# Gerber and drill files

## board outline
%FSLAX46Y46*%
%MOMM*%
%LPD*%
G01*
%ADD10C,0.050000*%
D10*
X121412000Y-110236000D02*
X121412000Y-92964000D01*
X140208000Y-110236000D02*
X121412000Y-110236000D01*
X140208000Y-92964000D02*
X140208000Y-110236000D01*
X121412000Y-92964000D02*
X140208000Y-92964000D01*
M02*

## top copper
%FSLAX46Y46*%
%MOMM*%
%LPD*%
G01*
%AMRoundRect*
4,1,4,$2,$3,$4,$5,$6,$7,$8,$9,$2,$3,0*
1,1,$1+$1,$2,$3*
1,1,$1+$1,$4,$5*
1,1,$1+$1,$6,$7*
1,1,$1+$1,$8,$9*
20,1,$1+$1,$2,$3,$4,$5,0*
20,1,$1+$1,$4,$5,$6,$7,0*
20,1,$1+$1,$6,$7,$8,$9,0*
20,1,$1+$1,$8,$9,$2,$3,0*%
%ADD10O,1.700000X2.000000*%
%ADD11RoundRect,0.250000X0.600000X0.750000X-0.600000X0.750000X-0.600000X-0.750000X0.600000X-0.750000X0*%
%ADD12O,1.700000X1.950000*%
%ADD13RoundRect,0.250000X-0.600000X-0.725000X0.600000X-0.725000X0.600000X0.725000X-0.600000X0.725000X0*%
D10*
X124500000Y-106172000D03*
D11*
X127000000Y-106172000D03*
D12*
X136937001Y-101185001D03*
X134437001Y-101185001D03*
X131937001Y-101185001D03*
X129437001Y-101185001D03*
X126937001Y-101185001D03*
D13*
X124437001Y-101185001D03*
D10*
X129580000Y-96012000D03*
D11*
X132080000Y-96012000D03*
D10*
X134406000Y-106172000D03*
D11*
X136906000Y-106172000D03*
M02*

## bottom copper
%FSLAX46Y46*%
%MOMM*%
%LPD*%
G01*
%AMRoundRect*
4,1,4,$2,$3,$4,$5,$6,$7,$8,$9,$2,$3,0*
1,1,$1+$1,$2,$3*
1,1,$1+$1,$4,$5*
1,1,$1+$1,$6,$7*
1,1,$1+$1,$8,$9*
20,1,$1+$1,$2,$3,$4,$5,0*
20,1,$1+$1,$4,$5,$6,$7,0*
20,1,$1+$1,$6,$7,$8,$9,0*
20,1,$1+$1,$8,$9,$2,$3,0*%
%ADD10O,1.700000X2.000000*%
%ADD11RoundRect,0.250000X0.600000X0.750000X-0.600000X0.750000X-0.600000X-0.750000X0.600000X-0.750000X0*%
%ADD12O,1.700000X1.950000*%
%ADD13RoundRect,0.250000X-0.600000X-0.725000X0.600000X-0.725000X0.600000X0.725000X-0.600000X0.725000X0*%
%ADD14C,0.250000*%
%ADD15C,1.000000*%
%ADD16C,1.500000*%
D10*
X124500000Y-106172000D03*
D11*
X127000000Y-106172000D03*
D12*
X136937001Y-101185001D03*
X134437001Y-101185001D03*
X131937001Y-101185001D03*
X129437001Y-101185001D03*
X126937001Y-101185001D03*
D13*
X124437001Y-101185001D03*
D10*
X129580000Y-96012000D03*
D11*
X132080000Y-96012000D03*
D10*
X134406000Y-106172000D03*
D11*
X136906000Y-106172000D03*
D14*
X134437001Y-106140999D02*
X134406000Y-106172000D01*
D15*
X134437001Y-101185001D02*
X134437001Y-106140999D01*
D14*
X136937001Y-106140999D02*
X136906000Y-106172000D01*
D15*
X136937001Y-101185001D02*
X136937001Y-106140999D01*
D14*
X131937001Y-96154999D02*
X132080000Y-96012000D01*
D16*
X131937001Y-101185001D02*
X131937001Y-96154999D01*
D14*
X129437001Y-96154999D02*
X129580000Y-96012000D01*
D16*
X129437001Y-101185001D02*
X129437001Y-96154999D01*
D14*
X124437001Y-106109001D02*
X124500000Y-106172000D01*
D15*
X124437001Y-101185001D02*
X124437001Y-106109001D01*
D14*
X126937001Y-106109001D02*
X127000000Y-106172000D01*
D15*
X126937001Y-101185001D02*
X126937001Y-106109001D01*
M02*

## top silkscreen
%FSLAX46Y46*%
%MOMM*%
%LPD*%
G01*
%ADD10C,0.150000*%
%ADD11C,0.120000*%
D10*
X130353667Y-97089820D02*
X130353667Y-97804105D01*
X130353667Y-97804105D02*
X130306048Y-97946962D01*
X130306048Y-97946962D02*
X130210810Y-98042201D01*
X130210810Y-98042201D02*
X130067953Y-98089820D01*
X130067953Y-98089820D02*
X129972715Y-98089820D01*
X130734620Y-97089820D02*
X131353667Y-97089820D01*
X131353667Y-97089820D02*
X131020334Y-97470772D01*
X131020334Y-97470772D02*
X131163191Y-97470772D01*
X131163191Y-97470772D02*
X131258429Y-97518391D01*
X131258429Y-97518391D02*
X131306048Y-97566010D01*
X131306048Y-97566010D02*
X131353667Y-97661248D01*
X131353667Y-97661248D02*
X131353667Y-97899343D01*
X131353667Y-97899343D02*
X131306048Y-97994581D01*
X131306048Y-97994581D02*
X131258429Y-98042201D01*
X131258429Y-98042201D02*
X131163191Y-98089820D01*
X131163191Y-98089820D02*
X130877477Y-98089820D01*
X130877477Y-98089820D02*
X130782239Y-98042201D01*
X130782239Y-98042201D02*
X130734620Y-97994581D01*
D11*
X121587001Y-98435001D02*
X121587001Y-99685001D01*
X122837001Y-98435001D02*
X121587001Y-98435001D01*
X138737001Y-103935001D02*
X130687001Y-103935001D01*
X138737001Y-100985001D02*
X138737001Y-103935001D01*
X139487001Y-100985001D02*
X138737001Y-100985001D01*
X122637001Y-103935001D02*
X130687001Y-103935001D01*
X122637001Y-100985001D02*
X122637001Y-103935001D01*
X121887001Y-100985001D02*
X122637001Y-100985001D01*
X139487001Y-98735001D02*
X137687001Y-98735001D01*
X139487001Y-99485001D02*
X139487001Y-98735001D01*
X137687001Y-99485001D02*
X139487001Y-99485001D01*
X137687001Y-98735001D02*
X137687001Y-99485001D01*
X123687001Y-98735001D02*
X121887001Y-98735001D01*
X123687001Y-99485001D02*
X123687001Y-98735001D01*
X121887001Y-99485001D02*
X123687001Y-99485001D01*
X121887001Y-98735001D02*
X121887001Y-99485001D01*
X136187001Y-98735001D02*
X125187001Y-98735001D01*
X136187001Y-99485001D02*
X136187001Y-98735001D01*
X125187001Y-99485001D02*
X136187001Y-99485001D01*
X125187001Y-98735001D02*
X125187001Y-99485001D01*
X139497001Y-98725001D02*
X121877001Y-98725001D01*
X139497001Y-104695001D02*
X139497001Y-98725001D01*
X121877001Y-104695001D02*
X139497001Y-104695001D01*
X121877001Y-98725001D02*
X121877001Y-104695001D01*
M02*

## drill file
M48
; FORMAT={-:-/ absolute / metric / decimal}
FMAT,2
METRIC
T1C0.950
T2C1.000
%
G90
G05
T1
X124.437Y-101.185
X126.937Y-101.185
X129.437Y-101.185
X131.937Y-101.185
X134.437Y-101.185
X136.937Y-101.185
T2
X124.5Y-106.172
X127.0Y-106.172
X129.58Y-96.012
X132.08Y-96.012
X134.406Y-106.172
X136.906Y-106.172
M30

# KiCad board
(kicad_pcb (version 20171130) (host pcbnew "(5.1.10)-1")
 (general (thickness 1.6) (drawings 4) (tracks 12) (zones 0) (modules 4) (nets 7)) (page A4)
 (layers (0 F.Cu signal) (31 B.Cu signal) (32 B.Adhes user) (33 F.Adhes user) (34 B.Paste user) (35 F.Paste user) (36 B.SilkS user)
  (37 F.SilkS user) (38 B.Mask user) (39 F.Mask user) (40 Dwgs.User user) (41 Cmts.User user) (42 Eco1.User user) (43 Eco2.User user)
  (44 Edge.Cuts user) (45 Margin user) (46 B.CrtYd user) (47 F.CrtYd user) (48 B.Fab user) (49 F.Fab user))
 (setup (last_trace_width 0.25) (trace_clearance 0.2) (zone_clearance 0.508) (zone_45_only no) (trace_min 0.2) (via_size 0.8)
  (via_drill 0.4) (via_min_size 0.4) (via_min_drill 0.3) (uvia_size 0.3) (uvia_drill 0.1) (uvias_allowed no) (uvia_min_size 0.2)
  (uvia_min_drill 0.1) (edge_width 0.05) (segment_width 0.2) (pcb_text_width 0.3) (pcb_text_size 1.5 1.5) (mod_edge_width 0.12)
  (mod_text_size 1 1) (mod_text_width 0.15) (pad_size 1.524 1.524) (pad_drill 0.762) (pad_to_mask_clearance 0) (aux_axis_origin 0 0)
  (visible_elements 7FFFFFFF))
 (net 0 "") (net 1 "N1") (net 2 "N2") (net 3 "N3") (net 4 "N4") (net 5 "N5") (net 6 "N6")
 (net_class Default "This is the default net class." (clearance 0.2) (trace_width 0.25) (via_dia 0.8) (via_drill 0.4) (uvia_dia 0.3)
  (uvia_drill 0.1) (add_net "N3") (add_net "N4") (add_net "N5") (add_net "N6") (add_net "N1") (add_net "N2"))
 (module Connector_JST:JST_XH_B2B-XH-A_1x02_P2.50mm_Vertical (layer B.Cu) (at 127 106.172 180)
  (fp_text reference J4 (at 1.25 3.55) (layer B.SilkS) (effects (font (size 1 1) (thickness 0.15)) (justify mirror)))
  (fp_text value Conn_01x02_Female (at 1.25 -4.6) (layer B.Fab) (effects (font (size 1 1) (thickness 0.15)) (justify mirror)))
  (pad 2 thru_hole oval (at 2.5 0 180) (size 1.7 2) (drill 1) (layers *.Cu *.Mask) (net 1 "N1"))
  (pad 1 thru_hole roundrect (at 0 0 180) (size 1.7 2) (drill 1) (layers *.Cu *.Mask) (roundrect_rratio 0.1470588235294118) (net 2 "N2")))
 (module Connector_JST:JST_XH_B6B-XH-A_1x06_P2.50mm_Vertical (layer F.Cu) (at 124.437001 101.185001)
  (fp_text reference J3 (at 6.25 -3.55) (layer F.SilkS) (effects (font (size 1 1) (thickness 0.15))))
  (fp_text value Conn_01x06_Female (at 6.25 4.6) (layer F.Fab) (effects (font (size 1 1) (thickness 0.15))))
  (fp_line (start -2.85 -2.75) (end -2.85 -1.5) (layer F.SilkS) (width 0.12))
  (fp_line (start -1.6 -2.75) (end -2.85 -2.75) (layer F.SilkS) (width 0.12))
  (fp_line (start 14.3 2.75) (end 6.25 2.75) (layer F.SilkS) (width 0.12))
  (fp_line (start 14.3 -0.2) (end 14.3 2.75) (layer F.SilkS) (width 0.12))
  (fp_line (start 15.05 -0.2) (end 14.3 -0.2) (layer F.SilkS) (width 0.12))
  (fp_line (start -1.8 2.75) (end 6.25 2.75) (layer F.SilkS) (width 0.12))
  (fp_line (start -1.8 -0.2) (end -1.8 2.75) (layer F.SilkS) (width 0.12))
  (fp_line (start -2.55 -0.2) (end -1.8 -0.2) (layer F.SilkS) (width 0.12))
  (fp_line (start 15.05 -2.45) (end 13.25 -2.45) (layer F.SilkS) (width 0.12))
  (fp_line (start 15.05 -1.7) (end 15.05 -2.45) (layer F.SilkS) (width 0.12))
  (fp_line (start 13.25 -1.7) (end 15.05 -1.7) (layer F.SilkS) (width 0.12))
  (fp_line (start 13.25 -2.45) (end 13.25 -1.7) (layer F.SilkS) (width 0.12))
  (fp_line (start -0.75 -2.45) (end -2.55 -2.45) (layer F.SilkS) (width 0.12))
  (fp_line (start -0.75 -1.7) (end -0.75 -2.45) (layer F.SilkS) (width 0.12))
  (fp_line (start -2.55 -1.7) (end -0.75 -1.7) (layer F.SilkS) (width 0.12))
  (fp_line (start -2.55 -2.45) (end -2.55 -1.7) (layer F.SilkS) (width 0.12))
  (fp_line (start 11.75 -2.45) (end 0.75 -2.45) (layer F.SilkS) (width 0.12))
  (fp_line (start 11.75 -1.7) (end 11.75 -2.45) (layer F.SilkS) (width 0.12))
  (fp_line (start 0.75 -1.7) (end 11.75 -1.7) (layer F.SilkS) (width 0.12))
  (fp_line (start 0.75 -2.45) (end 0.75 -1.7) (layer F.SilkS) (width 0.12))
  (fp_line (start 15.06 -2.46) (end -2.56 -2.46) (layer F.SilkS) (width 0.12))
  (fp_line (start 15.06 3.51) (end 15.06 -2.46) (layer F.SilkS) (width 0.12))
  (fp_line (start -2.56 3.51) (end 15.06 3.51) (layer F.SilkS) (width 0.12))
  (fp_line (start -2.56 -2.46) (end -2.56 3.51) (layer F.SilkS) (width 0.12))
  (pad 6 thru_hole oval (at 12.5 0) (size 1.7 1.95) (drill 0.95) (layers *.Cu *.Mask) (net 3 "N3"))
  (pad 5 thru_hole oval (at 10 0) (size 1.7 1.95) (drill 0.95) (layers *.Cu *.Mask) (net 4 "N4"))
  (pad 4 thru_hole oval (at 7.5 0) (size 1.7 1.95) (drill 0.95) (layers *.Cu *.Mask) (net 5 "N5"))
  (pad 3 thru_hole oval (at 5 0) (size 1.7 1.95) (drill 0.95) (layers *.Cu *.Mask) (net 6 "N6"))
  (pad 2 thru_hole oval (at 2.5 0) (size 1.7 1.95) (drill 0.95) (layers *.Cu *.Mask) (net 2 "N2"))
  (pad 1 thru_hole roundrect (at 0 0) (size 1.7 1.95) (drill 0.95) (layers *.Cu *.Mask) (roundrect_rratio 0.1470588235294118) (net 1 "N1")))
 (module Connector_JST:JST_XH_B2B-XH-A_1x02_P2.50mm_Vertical (layer B.Cu) (at 132.08 96.012 180)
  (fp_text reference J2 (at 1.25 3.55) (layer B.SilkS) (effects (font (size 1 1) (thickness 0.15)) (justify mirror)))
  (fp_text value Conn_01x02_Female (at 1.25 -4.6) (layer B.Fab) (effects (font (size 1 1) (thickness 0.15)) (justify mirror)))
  (pad 2 thru_hole oval (at 2.5 0 180) (size 1.7 2) (drill 1) (layers *.Cu *.Mask) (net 6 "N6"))
  (pad 1 thru_hole roundrect (at 0 0 180) (size 1.7 2) (drill 1) (layers *.Cu *.Mask) (roundrect_rratio 0.1470588235294118) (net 5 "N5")))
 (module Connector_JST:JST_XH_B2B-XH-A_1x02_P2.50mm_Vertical (layer B.Cu) (at 136.906 106.172 180)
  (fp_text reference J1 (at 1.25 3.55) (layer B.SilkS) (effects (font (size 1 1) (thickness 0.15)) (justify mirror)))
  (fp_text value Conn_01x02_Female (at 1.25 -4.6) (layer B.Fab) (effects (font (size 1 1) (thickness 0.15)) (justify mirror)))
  (pad 2 thru_hole oval (at 2.5 0 180) (size 1.7 2) (drill 1) (layers *.Cu *.Mask) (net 4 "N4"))
  (pad 1 thru_hole roundrect (at 0 0 180) (size 1.7 2) (drill 1) (layers *.Cu *.Mask) (roundrect_rratio 0.1470588235294118) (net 3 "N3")))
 (gr_line (start 121.412 110.236) (end 121.412 92.964) (layer Edge.Cuts) (width 0.05))
 (gr_line (start 140.208 110.236) (end 121.412 110.236) (layer Edge.Cuts) (width 0.05))
 (gr_line (start 140.208 92.964) (end 140.208 110.236) (layer Edge.Cuts) (width 0.05))
 (gr_line (start 121.412 92.964) (end 140.208 92.964) (layer Edge.Cuts) (width 0.05))
 (segment (start 134.437001 106.140999) (end 134.406 106.172) (width 0.25) (layer B.Cu) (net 4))
 (segment (start 134.437001 101.185001) (end 134.437001 106.140999) (width 1) (layer B.Cu) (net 4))
 (segment (start 136.937001 106.140999) (end 136.906 106.172) (width 0.25) (layer B.Cu) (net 3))
 (segment (start 136.937001 101.185001) (end 136.937001 106.140999) (width 1) (layer B.Cu) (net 3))
 (segment (start 131.937001 96.154999) (end 132.08 96.012) (width 0.25) (layer B.Cu) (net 5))
 (segment (start 131.937001 101.185001) (end 131.937001 96.154999) (width 1.5) (layer B.Cu) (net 5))
 (segment (start 129.437001 96.154999) (end 129.58 96.012) (width 0.25) (layer B.Cu) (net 6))
 (segment (start 129.437001 101.185001) (end 129.437001 96.154999) (width 1.5) (layer B.Cu) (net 6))
 (segment (start 124.437001 106.109001) (end 124.5 106.172) (width 0.25) (layer B.Cu) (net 1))
 (segment (start 124.437001 101.185001) (end 124.437001 106.109001) (width 1) (layer B.Cu) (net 1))
 (segment (start 126.937001 106.109001) (end 127 106.172) (width 0.25) (layer B.Cu) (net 2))
 (segment (start 126.937001 101.185001) (end 126.937001 106.109001) (width 1) (layer B.Cu) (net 2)))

